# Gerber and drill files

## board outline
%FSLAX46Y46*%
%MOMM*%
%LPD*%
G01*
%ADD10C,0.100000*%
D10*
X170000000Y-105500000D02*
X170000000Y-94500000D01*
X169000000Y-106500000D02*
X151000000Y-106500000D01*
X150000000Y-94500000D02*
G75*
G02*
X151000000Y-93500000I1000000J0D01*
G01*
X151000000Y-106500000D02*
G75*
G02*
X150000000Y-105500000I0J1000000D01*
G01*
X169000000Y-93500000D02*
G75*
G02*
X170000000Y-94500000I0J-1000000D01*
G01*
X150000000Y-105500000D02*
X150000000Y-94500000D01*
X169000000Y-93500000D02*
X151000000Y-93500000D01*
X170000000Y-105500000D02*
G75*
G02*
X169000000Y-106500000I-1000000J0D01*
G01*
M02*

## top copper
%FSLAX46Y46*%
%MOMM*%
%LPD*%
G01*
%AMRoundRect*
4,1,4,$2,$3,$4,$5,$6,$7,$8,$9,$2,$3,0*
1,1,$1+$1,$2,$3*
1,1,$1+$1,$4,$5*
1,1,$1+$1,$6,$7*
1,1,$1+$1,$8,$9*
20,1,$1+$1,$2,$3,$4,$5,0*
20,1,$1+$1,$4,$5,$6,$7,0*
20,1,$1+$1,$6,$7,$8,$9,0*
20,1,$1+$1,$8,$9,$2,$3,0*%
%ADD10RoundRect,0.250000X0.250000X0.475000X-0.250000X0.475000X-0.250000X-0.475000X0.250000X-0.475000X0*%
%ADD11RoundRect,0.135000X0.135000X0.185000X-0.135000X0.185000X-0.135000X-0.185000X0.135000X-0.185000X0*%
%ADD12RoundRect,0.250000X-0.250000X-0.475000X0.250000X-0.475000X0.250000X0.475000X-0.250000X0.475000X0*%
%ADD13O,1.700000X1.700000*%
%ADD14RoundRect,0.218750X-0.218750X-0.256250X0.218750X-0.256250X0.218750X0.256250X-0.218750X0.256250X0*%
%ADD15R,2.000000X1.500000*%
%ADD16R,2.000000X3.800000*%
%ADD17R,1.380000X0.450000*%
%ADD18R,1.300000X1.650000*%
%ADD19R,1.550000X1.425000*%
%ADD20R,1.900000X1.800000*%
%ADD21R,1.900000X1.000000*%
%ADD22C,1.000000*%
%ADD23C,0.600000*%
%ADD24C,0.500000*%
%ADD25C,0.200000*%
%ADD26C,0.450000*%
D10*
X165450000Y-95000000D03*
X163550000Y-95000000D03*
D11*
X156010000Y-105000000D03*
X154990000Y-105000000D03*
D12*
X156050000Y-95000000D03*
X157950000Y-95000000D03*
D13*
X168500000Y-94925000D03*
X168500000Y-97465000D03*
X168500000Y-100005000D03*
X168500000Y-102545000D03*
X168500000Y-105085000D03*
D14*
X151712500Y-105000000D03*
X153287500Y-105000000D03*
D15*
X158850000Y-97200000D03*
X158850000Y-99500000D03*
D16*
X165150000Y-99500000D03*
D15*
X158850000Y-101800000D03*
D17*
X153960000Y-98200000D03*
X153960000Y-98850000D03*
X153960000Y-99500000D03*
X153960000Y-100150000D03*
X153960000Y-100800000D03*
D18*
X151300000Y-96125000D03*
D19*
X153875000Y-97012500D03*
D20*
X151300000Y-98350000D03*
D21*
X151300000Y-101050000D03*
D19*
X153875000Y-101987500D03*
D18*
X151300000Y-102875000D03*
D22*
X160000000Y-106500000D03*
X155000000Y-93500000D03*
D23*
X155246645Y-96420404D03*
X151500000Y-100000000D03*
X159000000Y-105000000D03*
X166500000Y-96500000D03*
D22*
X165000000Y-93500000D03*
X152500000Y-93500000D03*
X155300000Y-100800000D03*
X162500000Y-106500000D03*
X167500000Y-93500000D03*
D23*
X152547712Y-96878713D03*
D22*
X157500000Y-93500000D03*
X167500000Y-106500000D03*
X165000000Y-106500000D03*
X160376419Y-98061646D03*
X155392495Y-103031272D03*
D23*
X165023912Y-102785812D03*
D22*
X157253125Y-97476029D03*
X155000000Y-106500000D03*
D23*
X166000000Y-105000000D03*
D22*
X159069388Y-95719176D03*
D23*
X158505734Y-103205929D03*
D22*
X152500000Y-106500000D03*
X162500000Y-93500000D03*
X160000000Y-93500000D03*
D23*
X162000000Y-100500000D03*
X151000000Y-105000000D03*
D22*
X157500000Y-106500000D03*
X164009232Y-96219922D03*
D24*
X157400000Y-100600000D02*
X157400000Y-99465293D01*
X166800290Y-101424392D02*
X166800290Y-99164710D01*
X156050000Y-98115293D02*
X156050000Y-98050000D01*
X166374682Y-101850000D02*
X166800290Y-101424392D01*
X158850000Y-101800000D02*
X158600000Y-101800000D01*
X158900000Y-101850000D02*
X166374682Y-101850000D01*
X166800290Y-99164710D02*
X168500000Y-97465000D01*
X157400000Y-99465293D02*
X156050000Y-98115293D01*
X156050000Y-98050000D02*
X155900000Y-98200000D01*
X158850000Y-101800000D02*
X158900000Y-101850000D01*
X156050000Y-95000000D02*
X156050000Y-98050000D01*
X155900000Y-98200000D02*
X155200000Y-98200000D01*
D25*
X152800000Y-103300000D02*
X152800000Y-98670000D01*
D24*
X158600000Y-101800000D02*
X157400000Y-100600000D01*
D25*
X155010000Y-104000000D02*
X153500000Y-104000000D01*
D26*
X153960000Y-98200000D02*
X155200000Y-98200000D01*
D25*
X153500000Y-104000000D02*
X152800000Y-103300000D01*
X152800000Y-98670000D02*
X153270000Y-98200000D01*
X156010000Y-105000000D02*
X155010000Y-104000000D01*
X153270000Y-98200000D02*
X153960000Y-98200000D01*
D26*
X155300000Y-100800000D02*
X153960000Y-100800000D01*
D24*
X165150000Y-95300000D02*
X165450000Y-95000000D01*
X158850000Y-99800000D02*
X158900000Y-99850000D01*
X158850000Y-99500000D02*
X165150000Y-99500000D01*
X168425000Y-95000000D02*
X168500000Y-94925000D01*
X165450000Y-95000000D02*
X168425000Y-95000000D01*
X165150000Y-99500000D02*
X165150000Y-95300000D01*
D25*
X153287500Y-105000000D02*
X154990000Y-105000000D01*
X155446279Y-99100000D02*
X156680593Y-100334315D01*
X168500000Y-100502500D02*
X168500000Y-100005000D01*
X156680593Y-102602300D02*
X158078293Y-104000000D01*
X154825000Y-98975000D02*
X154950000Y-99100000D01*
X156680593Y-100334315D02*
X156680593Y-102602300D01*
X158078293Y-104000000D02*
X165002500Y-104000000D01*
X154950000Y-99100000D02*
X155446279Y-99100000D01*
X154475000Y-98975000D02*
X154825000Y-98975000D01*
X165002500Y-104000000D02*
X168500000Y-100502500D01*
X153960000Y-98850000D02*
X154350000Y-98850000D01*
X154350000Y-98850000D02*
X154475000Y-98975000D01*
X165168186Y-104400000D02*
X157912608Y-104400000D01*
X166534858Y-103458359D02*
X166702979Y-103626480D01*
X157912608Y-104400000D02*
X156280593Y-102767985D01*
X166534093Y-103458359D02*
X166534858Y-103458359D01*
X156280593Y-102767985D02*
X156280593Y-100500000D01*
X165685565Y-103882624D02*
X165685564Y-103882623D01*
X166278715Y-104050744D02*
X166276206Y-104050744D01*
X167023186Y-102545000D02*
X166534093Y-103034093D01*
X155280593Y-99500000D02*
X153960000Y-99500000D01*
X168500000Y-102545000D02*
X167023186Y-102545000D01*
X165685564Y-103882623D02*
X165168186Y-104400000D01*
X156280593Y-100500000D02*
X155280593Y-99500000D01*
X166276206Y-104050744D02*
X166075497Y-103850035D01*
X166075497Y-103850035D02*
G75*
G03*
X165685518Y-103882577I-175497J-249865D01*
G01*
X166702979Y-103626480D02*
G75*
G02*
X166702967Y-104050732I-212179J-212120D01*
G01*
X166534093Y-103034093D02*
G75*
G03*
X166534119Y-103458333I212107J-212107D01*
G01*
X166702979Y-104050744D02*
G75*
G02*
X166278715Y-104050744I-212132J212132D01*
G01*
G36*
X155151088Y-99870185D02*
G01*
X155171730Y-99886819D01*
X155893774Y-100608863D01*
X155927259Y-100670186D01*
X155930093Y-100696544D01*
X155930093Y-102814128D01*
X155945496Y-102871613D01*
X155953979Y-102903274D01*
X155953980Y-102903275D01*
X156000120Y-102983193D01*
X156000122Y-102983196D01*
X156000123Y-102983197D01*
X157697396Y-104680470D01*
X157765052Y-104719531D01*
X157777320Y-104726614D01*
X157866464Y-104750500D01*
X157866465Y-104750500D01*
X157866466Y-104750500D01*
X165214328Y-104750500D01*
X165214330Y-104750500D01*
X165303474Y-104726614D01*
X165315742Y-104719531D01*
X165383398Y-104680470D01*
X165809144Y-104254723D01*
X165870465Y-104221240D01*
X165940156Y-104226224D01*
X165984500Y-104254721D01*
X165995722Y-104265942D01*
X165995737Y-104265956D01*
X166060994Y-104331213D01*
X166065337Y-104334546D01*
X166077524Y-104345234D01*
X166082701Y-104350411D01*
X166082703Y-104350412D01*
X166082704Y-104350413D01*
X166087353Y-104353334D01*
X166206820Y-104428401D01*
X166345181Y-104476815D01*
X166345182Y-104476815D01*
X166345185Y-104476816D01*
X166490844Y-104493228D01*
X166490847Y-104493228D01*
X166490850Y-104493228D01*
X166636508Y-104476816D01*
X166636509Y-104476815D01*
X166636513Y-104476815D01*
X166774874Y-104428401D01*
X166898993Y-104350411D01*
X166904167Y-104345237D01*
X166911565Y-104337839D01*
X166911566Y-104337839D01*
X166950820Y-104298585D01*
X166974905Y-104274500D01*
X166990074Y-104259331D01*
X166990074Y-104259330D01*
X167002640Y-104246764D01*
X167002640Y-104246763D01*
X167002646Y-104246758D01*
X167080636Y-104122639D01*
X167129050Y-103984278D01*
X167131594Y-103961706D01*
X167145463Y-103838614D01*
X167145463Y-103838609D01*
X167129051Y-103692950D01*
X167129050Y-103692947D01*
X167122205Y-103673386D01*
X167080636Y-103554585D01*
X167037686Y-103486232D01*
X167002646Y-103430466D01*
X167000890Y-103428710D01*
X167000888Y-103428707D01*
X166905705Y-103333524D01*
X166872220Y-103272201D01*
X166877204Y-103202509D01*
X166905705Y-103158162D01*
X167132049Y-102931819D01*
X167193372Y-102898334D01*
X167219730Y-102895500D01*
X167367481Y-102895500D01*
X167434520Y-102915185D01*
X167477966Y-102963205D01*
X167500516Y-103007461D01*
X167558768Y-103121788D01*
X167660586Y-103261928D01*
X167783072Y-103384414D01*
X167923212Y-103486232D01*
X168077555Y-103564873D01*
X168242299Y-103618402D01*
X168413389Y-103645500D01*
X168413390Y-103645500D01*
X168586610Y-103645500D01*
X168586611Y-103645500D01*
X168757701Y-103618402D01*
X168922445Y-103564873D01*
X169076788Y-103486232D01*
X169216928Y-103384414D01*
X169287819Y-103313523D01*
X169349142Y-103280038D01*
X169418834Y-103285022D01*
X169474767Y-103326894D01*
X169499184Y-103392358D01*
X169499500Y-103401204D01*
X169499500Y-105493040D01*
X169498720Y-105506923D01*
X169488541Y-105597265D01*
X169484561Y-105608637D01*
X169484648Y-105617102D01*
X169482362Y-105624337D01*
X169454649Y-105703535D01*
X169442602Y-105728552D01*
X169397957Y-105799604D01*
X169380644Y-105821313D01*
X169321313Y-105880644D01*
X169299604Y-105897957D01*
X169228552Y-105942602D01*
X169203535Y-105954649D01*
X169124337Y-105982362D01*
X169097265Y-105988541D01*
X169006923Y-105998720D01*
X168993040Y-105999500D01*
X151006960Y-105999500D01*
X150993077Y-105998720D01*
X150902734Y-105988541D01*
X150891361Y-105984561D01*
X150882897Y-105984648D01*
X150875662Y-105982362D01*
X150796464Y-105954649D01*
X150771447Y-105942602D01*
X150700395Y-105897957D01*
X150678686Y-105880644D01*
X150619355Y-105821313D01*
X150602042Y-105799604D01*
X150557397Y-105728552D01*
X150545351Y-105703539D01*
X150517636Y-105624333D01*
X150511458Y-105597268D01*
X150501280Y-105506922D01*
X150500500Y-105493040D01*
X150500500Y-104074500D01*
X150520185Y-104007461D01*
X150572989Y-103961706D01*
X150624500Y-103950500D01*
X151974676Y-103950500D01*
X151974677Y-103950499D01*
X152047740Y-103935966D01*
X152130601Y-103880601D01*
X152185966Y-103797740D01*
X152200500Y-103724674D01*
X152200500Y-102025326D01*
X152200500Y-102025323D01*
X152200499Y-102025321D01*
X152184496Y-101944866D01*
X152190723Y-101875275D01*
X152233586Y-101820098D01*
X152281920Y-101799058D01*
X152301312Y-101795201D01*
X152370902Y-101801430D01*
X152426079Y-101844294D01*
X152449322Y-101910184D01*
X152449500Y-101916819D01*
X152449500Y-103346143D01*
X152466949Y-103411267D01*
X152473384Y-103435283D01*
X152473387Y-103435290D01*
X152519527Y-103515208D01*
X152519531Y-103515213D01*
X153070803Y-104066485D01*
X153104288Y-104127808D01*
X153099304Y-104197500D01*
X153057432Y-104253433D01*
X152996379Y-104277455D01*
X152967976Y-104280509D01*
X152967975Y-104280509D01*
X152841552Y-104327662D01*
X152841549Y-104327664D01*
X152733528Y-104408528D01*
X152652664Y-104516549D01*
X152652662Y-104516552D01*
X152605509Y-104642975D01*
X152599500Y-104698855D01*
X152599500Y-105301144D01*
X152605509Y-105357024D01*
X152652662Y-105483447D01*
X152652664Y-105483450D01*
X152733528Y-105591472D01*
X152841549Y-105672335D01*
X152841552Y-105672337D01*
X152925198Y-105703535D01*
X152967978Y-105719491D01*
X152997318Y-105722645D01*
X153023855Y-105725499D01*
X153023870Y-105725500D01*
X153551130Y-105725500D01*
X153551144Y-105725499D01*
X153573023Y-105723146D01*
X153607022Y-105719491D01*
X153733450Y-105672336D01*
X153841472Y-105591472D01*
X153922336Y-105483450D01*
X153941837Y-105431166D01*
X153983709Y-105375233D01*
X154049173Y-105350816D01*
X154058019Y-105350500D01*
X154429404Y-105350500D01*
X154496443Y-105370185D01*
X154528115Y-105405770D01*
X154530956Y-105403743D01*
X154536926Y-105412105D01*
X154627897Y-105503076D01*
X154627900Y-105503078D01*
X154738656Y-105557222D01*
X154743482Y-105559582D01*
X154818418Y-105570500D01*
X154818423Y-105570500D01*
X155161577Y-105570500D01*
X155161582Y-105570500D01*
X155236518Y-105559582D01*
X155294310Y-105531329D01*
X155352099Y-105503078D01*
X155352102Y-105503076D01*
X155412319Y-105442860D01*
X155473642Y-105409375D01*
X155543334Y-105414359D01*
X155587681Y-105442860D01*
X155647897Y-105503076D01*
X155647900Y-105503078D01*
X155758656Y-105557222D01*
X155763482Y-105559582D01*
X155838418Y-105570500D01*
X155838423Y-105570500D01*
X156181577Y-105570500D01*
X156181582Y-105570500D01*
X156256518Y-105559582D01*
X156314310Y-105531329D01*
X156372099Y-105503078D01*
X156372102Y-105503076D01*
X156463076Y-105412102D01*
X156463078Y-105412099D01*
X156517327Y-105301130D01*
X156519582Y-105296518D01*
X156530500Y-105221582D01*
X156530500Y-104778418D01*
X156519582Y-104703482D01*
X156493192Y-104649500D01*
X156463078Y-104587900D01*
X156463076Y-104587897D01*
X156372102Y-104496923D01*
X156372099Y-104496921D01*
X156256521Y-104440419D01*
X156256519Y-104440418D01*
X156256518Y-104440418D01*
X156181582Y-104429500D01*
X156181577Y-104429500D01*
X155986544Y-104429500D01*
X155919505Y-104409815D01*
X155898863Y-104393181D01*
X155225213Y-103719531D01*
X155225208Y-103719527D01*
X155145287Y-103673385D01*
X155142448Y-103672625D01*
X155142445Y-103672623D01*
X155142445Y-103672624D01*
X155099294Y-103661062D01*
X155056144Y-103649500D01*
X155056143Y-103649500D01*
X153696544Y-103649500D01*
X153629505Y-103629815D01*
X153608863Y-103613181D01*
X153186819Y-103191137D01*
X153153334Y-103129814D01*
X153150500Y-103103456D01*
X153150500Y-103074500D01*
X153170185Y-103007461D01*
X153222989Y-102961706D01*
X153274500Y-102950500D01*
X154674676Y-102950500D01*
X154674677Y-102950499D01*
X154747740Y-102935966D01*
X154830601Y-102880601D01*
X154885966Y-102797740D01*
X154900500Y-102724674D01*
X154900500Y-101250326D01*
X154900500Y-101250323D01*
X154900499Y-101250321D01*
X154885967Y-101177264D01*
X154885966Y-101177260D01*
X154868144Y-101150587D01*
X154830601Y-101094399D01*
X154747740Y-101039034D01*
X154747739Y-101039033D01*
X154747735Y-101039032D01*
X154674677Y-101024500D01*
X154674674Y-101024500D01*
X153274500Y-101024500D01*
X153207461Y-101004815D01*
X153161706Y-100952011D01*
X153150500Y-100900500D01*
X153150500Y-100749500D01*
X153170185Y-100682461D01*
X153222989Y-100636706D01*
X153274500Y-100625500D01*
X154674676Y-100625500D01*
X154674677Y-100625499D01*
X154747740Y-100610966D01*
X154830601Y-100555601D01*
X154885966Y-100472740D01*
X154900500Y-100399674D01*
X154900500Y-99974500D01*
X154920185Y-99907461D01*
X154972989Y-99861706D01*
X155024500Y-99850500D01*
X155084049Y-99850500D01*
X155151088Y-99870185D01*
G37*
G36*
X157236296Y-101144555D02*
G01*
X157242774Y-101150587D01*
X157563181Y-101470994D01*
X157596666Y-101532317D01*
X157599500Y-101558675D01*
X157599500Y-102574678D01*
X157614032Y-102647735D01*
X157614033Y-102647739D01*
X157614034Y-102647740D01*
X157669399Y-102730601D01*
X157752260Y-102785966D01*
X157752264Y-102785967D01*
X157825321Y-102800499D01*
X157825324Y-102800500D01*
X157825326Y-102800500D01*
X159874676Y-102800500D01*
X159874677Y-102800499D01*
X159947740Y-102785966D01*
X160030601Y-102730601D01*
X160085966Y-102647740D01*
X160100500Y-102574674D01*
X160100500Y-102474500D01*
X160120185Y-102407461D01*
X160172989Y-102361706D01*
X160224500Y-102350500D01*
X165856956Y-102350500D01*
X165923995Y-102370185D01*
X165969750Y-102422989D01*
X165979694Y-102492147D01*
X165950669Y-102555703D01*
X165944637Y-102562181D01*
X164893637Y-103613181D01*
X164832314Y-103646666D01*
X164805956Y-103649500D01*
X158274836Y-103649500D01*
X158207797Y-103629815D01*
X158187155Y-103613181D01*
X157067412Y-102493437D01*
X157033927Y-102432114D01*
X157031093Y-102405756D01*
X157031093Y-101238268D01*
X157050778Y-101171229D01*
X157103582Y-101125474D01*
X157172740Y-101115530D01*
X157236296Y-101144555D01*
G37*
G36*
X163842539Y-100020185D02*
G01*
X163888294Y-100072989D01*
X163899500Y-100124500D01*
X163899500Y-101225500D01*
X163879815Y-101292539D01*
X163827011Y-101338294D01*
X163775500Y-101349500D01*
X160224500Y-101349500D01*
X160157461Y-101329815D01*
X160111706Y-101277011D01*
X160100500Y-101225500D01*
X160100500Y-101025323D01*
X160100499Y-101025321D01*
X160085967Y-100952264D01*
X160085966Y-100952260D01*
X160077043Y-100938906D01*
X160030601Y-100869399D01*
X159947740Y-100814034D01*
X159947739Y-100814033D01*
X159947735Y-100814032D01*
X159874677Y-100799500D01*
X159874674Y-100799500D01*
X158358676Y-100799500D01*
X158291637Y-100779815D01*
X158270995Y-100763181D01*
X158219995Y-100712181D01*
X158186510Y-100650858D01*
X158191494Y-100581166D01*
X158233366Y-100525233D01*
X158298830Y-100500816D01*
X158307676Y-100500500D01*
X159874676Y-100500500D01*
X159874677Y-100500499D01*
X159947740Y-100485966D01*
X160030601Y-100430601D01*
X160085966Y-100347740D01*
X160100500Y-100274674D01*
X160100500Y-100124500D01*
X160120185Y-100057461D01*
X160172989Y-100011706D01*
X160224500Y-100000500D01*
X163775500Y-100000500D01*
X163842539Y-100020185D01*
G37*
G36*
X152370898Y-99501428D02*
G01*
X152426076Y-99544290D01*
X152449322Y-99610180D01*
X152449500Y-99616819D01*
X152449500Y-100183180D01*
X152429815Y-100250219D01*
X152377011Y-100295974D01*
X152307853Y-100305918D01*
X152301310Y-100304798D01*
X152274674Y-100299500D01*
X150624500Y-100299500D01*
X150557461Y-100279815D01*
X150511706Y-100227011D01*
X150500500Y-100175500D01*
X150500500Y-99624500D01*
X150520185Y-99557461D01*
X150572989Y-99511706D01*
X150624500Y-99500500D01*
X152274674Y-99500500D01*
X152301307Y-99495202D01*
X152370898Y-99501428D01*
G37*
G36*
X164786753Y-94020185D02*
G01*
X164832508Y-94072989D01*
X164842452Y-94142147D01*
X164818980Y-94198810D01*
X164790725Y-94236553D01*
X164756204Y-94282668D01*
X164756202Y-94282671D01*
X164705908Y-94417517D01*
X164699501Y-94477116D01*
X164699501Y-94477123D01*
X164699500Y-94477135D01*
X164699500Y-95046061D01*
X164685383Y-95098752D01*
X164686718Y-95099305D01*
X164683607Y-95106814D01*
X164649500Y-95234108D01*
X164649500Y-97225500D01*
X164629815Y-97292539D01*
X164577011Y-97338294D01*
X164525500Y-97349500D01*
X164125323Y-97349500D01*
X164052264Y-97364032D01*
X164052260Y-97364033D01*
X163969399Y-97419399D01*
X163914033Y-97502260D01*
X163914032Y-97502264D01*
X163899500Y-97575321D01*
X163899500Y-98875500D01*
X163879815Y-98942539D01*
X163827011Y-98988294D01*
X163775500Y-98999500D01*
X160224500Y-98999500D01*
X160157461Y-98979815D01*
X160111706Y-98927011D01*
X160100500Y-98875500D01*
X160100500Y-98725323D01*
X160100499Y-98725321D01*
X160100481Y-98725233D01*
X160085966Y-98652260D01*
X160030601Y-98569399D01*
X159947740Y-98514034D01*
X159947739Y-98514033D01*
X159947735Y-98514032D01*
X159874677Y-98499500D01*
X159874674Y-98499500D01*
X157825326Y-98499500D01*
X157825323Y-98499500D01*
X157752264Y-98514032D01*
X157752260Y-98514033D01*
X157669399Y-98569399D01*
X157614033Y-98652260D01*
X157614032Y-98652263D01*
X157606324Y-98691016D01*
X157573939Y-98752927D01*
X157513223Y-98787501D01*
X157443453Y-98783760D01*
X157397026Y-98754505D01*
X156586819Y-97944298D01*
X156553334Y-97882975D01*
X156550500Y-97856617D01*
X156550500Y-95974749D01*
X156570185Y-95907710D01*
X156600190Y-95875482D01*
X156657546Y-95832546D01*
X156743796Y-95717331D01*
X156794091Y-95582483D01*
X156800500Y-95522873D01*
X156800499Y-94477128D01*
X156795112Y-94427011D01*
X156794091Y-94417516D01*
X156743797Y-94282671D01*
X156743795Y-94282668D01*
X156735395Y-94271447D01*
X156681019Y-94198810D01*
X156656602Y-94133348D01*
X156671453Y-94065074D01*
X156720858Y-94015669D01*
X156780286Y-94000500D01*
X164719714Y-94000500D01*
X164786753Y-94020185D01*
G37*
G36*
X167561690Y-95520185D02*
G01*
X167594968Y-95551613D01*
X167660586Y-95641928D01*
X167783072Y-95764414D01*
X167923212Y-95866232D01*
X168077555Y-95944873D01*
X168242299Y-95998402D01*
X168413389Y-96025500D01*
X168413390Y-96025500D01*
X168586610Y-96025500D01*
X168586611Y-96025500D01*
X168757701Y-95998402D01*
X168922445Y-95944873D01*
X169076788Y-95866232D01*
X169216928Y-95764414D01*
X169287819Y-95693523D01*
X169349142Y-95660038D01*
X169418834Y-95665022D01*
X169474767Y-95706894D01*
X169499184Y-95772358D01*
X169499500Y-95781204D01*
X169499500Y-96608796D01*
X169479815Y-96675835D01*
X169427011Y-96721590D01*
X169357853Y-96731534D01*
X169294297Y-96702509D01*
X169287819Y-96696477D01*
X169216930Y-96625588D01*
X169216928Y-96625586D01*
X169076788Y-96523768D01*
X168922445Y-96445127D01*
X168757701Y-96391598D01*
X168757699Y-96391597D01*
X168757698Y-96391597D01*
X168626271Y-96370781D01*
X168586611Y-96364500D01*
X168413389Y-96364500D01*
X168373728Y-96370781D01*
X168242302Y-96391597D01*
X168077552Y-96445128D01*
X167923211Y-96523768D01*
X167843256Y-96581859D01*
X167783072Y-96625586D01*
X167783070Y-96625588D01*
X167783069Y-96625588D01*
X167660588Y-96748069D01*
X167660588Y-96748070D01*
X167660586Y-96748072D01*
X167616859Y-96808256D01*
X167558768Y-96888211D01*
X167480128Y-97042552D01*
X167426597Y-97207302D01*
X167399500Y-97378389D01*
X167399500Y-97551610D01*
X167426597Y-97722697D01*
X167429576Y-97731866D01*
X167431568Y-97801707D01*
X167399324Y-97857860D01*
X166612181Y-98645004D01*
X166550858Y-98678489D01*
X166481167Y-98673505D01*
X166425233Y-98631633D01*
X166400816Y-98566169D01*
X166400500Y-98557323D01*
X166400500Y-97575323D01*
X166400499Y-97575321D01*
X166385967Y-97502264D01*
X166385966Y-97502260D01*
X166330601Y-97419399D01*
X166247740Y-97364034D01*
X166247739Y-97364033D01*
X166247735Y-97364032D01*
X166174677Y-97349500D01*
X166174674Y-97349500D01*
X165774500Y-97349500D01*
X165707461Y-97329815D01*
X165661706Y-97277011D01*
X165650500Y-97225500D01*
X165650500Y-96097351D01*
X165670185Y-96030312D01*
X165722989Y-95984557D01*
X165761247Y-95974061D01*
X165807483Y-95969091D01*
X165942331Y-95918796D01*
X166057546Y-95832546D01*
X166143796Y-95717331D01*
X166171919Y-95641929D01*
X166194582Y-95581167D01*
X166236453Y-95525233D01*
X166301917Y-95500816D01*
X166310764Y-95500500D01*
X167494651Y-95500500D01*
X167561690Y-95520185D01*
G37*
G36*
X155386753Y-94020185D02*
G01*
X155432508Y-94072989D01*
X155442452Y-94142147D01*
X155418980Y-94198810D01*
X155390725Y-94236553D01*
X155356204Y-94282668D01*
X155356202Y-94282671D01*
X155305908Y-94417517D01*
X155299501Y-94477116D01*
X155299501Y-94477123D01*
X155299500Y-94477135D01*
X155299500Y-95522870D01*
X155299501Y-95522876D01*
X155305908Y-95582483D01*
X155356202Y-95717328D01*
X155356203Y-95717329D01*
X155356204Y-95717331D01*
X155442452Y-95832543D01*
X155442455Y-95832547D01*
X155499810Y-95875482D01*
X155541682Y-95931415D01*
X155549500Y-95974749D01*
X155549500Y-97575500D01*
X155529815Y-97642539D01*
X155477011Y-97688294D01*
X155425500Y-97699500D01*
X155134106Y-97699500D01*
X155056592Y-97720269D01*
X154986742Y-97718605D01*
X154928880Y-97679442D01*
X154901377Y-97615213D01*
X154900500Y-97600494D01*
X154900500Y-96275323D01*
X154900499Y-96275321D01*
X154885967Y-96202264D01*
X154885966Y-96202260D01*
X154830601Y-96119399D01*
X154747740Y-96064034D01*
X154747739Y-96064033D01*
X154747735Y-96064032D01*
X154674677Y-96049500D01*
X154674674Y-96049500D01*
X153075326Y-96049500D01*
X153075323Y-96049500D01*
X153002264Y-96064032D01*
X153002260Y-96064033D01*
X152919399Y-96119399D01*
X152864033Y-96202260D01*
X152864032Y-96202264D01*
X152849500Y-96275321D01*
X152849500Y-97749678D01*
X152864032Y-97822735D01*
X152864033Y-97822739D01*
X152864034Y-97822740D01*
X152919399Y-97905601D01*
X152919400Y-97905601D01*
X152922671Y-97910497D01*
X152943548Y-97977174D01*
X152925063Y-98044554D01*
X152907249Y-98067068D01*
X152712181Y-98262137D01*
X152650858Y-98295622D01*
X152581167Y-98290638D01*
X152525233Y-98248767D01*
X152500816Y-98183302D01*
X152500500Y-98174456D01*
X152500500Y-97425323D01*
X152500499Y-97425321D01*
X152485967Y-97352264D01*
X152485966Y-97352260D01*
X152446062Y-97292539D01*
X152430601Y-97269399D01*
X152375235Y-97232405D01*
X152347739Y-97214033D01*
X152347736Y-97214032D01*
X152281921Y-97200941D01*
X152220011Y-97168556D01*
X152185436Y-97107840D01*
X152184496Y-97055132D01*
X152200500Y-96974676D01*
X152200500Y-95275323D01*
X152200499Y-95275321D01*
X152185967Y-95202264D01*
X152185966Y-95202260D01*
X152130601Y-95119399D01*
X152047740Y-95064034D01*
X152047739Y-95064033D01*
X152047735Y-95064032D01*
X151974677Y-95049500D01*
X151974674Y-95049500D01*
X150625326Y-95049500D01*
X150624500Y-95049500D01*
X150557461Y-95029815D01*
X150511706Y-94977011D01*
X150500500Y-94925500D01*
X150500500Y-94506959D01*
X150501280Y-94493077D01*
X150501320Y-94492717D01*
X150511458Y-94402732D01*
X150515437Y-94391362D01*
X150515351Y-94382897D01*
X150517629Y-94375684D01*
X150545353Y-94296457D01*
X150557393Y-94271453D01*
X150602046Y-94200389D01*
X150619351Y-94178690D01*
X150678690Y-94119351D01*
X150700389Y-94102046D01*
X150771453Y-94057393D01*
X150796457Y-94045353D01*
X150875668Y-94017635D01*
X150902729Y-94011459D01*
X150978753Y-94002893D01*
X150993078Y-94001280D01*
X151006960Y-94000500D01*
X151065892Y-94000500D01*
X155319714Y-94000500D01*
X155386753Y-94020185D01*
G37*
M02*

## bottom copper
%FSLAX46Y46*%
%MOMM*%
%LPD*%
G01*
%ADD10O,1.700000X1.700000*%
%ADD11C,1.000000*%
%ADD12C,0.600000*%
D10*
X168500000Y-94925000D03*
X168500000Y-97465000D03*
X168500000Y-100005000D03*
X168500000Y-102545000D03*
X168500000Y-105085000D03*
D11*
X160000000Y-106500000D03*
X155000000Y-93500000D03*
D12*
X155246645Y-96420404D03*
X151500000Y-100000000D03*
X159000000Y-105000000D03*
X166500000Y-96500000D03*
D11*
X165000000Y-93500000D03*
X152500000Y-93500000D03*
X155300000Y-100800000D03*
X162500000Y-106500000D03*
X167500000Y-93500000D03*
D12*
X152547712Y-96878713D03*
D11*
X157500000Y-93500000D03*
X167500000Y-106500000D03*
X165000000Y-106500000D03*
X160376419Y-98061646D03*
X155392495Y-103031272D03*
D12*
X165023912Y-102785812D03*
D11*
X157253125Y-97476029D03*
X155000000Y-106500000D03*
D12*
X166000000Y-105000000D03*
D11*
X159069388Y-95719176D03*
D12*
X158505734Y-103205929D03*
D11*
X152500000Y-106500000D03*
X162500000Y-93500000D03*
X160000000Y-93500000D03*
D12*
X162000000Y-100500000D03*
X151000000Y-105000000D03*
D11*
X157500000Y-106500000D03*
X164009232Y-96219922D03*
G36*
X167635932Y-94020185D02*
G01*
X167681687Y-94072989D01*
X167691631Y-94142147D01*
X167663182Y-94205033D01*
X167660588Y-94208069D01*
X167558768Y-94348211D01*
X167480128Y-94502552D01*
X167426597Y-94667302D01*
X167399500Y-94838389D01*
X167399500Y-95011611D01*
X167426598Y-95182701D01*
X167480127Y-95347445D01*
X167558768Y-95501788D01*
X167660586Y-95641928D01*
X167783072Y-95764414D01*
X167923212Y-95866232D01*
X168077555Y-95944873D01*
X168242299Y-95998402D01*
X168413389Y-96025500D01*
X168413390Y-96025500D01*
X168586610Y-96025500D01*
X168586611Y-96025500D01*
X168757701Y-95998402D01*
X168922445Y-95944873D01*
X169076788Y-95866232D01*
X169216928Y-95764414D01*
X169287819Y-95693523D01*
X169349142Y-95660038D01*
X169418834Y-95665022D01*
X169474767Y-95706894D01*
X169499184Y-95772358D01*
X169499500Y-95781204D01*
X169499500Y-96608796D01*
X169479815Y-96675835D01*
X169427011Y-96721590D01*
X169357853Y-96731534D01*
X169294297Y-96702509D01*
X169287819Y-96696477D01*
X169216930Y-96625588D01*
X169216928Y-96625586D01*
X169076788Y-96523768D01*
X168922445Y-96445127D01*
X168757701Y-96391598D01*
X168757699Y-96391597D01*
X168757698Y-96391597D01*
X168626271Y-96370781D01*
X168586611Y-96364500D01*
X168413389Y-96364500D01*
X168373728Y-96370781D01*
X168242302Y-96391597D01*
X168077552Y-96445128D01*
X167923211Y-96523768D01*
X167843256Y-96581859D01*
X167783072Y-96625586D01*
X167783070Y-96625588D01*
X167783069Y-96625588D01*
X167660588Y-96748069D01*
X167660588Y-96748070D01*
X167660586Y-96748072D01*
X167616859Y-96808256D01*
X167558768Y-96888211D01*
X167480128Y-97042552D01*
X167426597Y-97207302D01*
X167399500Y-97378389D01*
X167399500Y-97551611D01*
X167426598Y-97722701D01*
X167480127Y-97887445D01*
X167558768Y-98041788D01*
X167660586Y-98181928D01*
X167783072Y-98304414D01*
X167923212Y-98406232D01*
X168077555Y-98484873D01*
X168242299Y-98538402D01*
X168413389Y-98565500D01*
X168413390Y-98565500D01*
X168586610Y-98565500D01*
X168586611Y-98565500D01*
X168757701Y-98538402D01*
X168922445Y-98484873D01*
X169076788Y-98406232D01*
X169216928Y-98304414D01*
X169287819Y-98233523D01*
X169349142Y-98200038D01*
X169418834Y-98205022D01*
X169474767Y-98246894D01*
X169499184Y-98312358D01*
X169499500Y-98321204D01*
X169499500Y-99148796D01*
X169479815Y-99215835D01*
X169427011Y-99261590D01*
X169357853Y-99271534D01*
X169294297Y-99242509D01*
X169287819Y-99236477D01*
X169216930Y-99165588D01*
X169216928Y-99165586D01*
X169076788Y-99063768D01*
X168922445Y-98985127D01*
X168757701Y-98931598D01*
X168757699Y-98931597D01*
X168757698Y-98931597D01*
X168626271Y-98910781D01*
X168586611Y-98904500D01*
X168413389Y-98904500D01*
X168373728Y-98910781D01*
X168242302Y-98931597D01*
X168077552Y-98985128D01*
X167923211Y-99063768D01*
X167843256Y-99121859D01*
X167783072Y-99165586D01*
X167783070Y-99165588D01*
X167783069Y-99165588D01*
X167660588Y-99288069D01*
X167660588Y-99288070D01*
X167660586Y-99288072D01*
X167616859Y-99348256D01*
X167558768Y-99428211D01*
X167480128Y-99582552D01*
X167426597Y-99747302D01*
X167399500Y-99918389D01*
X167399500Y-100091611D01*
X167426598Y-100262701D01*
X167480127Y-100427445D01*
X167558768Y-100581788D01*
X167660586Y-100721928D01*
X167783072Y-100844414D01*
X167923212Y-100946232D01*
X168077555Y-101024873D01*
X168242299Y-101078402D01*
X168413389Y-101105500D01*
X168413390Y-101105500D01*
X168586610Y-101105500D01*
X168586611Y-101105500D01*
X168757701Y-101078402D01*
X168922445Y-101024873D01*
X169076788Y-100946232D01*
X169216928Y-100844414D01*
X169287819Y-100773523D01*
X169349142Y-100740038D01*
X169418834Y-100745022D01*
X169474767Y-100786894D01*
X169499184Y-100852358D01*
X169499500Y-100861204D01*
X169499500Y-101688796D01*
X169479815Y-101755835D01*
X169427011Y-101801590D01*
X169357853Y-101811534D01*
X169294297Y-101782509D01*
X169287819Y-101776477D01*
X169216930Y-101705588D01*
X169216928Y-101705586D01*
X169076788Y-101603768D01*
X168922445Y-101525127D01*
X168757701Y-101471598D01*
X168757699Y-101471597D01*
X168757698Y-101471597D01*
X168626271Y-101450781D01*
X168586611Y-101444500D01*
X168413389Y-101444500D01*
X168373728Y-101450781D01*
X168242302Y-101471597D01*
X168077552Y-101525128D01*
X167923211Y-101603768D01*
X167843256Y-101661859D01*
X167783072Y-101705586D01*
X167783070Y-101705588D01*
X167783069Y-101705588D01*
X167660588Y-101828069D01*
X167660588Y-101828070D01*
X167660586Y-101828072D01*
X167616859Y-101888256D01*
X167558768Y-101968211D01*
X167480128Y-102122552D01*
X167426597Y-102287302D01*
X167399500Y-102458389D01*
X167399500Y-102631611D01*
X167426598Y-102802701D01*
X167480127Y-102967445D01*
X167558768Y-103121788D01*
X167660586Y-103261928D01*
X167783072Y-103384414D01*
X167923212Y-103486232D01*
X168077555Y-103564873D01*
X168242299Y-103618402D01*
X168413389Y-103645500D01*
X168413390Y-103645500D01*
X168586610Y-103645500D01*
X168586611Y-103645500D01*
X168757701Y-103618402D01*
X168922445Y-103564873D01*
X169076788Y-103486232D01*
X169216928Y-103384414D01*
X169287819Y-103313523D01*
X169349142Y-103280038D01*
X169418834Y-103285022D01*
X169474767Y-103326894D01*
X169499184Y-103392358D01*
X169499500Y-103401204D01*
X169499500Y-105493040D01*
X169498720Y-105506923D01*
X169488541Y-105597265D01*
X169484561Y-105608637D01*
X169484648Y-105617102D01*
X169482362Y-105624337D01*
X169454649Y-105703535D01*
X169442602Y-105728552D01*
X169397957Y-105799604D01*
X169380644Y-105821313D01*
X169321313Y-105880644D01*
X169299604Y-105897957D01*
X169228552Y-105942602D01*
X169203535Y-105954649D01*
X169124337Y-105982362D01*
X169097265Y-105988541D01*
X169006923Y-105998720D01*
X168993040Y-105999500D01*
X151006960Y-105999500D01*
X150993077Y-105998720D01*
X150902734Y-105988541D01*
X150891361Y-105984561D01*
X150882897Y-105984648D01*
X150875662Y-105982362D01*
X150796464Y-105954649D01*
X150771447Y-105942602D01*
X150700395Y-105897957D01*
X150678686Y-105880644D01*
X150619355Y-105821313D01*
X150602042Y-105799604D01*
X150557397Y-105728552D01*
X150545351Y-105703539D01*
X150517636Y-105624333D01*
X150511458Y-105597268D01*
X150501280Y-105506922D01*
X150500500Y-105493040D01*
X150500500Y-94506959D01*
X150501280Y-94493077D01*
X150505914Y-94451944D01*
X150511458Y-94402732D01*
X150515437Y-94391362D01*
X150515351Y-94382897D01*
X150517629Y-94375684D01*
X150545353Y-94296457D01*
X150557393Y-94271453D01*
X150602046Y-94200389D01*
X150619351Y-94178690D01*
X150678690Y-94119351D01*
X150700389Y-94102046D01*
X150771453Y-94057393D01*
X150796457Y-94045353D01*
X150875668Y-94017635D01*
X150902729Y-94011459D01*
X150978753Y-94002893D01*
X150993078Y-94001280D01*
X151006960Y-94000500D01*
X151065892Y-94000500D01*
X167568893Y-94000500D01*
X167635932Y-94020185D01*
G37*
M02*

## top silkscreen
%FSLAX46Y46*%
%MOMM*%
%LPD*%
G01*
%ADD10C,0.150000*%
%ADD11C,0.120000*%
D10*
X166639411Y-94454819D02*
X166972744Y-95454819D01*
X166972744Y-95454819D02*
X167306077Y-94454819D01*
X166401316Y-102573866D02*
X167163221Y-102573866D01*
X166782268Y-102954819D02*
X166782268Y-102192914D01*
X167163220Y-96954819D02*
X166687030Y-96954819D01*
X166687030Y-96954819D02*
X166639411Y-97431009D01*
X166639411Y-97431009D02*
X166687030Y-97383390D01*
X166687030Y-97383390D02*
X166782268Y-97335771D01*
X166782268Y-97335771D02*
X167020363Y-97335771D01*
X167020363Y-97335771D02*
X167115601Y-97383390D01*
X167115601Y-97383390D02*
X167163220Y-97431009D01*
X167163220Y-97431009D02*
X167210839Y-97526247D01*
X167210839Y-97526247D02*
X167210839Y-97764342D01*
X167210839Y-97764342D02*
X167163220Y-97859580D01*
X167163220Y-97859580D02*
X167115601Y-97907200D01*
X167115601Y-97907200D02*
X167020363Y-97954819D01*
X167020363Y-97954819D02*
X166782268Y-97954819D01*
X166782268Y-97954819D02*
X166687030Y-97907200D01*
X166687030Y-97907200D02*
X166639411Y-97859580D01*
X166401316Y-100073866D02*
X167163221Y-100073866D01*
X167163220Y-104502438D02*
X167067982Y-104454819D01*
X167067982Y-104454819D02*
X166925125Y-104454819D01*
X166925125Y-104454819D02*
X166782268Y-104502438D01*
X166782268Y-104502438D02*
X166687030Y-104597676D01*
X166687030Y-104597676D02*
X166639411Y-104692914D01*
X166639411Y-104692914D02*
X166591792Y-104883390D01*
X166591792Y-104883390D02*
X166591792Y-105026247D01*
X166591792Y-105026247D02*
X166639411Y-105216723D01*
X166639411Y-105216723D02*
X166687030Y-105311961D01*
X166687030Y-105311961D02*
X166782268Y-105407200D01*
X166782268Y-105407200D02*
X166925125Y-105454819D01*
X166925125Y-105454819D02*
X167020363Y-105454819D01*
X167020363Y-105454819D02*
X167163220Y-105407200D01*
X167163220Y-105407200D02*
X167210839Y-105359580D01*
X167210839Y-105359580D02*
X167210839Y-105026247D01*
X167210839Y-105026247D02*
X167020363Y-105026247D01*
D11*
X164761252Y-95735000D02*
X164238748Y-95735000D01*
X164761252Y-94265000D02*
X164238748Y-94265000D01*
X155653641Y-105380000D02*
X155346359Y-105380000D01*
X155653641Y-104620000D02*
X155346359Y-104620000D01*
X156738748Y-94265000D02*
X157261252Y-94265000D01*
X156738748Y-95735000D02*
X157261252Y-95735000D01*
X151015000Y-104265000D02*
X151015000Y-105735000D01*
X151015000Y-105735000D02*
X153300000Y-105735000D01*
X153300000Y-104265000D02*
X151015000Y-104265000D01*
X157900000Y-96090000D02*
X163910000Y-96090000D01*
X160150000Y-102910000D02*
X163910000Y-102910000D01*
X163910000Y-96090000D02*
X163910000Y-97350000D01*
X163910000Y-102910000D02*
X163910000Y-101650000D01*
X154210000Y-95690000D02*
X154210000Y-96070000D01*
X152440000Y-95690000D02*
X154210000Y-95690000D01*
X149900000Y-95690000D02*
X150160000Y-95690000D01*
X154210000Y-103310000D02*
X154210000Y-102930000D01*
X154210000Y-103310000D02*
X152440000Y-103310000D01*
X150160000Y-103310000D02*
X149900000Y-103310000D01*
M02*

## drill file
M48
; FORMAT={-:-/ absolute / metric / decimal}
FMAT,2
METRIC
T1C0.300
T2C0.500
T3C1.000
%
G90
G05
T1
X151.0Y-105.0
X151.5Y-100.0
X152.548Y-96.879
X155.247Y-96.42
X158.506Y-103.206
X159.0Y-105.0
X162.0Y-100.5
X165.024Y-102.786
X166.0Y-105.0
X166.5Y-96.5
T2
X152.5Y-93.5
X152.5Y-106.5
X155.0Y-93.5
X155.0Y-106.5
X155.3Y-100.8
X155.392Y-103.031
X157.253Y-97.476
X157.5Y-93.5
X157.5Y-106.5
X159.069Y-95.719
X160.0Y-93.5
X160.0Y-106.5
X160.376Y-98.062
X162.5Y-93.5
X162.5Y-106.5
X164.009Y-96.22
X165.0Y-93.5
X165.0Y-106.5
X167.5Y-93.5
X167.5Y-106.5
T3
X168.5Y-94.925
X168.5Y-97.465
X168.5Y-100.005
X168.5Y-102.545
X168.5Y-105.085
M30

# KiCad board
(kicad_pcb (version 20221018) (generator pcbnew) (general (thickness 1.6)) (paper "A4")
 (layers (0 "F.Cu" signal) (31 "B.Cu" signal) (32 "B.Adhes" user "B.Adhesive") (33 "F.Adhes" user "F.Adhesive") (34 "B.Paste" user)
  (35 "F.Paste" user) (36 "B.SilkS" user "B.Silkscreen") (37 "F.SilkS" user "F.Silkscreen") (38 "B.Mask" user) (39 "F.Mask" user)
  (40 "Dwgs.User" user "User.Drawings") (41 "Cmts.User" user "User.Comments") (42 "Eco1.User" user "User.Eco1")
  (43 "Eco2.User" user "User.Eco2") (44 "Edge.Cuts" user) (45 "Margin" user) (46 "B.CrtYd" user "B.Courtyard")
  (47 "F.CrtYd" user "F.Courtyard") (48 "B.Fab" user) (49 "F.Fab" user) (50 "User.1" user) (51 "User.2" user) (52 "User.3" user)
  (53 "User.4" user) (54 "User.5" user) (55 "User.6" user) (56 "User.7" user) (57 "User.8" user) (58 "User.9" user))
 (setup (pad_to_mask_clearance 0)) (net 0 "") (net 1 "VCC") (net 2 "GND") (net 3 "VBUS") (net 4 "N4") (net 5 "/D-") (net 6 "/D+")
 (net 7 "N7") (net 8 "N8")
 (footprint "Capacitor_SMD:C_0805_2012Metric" (layer "F.Cu") (at 164.5 95 180)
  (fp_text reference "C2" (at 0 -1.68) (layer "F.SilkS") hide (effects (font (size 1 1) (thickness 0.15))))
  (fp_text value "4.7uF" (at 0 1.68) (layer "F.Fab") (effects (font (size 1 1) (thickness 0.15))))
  (fp_line (start -0.261252 -0.735) (end 0.261252 -0.735) (stroke (width 0.12) (type solid)) (layer "F.SilkS"))
  (fp_line (start -0.261252 0.735) (end 0.261252 0.735) (stroke (width 0.12) (type solid)) (layer "F.SilkS"))
  (pad "1" smd roundrect (at -0.95 0 180) (size 1 1.45) (layers "F.Cu" "F.Paste" "F.Mask") (roundrect_rratio 0.25) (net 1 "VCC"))
  (pad "2" smd roundrect (at 0.95 0 180) (size 1 1.45) (layers "F.Cu" "F.Paste" "F.Mask") (roundrect_rratio 0.25) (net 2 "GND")))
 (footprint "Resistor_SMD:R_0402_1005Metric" (layer "F.Cu") (at 155.5 105 180)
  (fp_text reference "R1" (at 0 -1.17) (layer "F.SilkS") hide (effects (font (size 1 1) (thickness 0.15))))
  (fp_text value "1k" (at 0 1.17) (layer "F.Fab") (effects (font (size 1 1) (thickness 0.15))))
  (fp_line (start -0.153641 -0.38) (end 0.153641 -0.38) (stroke (width 0.12) (type solid)) (layer "F.SilkS"))
  (fp_line (start -0.153641 0.38) (end 0.153641 0.38) (stroke (width 0.12) (type solid)) (layer "F.SilkS"))
  (pad "1" smd roundrect (at -0.51 0 180) (size 0.54 0.64) (layers "F.Cu" "F.Paste" "F.Mask") (roundrect_rratio 0.25) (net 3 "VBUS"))
  (pad "2" smd roundrect (at 0.51 0 180) (size 0.54 0.64) (layers "F.Cu" "F.Paste" "F.Mask") (roundrect_rratio 0.25) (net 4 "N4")))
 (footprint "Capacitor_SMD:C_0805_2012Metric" (layer "F.Cu") (at 157 95)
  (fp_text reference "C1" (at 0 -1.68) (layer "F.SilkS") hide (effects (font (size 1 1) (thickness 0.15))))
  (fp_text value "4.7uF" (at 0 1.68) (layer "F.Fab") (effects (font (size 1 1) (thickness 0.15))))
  (fp_line (start -0.261252 -0.735) (end 0.261252 -0.735) (stroke (width 0.12) (type solid)) (layer "F.SilkS"))
  (fp_line (start -0.261252 0.735) (end 0.261252 0.735) (stroke (width 0.12) (type solid)) (layer "F.SilkS"))
  (pad "1" smd roundrect (at -0.95 0) (size 1 1.45) (layers "F.Cu" "F.Paste" "F.Mask") (roundrect_rratio 0.25) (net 3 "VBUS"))
  (pad "2" smd roundrect (at 0.95 0) (size 1 1.45) (layers "F.Cu" "F.Paste" "F.Mask") (roundrect_rratio 0.25) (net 2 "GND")))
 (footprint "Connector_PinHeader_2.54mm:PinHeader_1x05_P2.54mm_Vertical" (layer "F.Cu") (at 168.5 94.925)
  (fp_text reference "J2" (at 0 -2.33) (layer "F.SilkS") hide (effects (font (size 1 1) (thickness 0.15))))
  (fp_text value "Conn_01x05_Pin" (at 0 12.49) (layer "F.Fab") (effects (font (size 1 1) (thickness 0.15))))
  (pad "1" thru_hole oval (at 0 0) (size 1.7 1.7) (drill 1) (layers "*.Cu" "*.Mask") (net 1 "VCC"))
  (pad "2" thru_hole oval (at 0 2.54) (size 1.7 1.7) (drill 1) (layers "*.Cu" "*.Mask") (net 3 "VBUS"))
  (pad "3" thru_hole oval (at 0 5.08) (size 1.7 1.7) (drill 1) (layers "*.Cu" "*.Mask") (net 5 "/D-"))
  (pad "4" thru_hole oval (at 0 7.62) (size 1.7 1.7) (drill 1) (layers "*.Cu" "*.Mask") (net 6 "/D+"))
  (pad "5" thru_hole oval (at 0 10.16) (size 1.7 1.7) (drill 1) (layers "*.Cu" "*.Mask") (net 2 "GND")))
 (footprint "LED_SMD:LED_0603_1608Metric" (layer "F.Cu") (at 152.5 105)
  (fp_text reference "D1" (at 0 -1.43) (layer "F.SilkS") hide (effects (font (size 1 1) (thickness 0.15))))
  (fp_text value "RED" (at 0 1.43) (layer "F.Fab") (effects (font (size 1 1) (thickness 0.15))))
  (fp_line (start -1.485 -0.735) (end -1.485 0.735) (stroke (width 0.12) (type solid)) (layer "F.SilkS"))
  (fp_line (start -1.485 0.735) (end 0.8 0.735) (stroke (width 0.12) (type solid)) (layer "F.SilkS"))
  (fp_line (start 0.8 -0.735) (end -1.485 -0.735) (stroke (width 0.12) (type solid)) (layer "F.SilkS"))
  (pad "1" smd roundrect (at -0.7875 0) (size 0.875 0.95) (layers "F.Cu" "F.Paste" "F.Mask") (roundrect_rratio 0.25) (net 2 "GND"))
  (pad "2" smd roundrect (at 0.7875 0) (size 0.875 0.95) (layers "F.Cu" "F.Paste" "F.Mask") (roundrect_rratio 0.25) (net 4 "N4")))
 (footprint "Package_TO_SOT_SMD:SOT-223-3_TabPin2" (layer "F.Cu") (at 162 99.5)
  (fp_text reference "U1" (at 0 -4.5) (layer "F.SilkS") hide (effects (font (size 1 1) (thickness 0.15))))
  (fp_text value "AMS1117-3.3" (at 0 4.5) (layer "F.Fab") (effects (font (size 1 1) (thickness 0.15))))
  (fp_line (start -4.1 -3.41) (end 1.91 -3.41) (stroke (width 0.12) (type solid)) (layer "F.SilkS"))
  (fp_line (start -1.85 3.41) (end 1.91 3.41) (stroke (width 0.12) (type solid)) (layer "F.SilkS"))
  (fp_line (start 1.91 -3.41) (end 1.91 -2.15) (stroke (width 0.12) (type solid)) (layer "F.SilkS"))
  (fp_line (start 1.91 3.41) (end 1.91 2.15) (stroke (width 0.12) (type solid)) (layer "F.SilkS"))
  (pad "1" smd rect (at -3.15 -2.3) (size 2 1.5) (layers "F.Cu" "F.Paste" "F.Mask") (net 2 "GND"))
  (pad "2" smd rect (at -3.15 0) (size 2 1.5) (layers "F.Cu" "F.Paste" "F.Mask") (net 1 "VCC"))
  (pad "2" smd rect (at 3.15 0) (size 2 3.8) (layers "F.Cu" "F.Paste" "F.Mask") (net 1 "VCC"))
  (pad "3" smd rect (at -3.15 2.3) (size 2 1.5) (layers "F.Cu" "F.Paste" "F.Mask") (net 3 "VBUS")))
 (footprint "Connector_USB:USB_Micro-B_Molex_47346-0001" (layer "F.Cu") (at 152.5 99.5 -90)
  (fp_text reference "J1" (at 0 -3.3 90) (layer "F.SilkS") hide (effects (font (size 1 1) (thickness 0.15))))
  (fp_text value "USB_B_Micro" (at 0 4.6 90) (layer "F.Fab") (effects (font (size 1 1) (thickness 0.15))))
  (fp_line (start -3.81 -1.71) (end -3.43 -1.71) (stroke (width 0.12) (type solid)) (layer "F.SilkS"))
  (fp_line (start -3.81 0.06) (end -3.81 -1.71) (stroke (width 0.12) (type solid)) (layer "F.SilkS"))
  (fp_line (start -3.81 2.6) (end -3.81 2.34) (stroke (width 0.12) (type solid)) (layer "F.SilkS"))
  (fp_line (start 3.81 -1.71) (end 3.43 -1.71) (stroke (width 0.12) (type solid)) (layer "F.SilkS"))
  (fp_line (start 3.81 -1.71) (end 3.81 0.06) (stroke (width 0.12) (type solid)) (layer "F.SilkS"))
  (fp_line (start 3.81 2.34) (end 3.81 2.6) (stroke (width 0.12) (type solid)) (layer "F.SilkS"))
  (pad "1" smd rect (at -1.3 -1.46 270) (size 0.45 1.38) (layers "F.Cu" "F.Paste" "F.Mask") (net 3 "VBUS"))
  (pad "2" smd rect (at -0.65 -1.46 270) (size 0.45 1.38) (layers "F.Cu" "F.Paste" "F.Mask") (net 5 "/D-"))
  (pad "3" smd rect (at 0 -1.46 270) (size 0.45 1.38) (layers "F.Cu" "F.Paste" "F.Mask") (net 6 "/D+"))
  (pad "4" smd rect (at 0.65 -1.46 270) (size 0.45 1.38) (layers "F.Cu" "F.Paste" "F.Mask") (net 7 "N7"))
  (pad "5" smd rect (at 1.3 -1.46 270) (size 0.45 1.38) (layers "F.Cu" "F.Paste" "F.Mask") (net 2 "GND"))
  (pad "6" smd rect (at -3.375 1.2 270) (size 1.65 1.3) (layers "F.Cu" "F.Paste" "F.Mask") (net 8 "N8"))
  (pad "6" smd rect (at -2.4875 -1.375 270) (size 1.425 1.55) (layers "F.Cu" "F.Paste" "F.Mask") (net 8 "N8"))
  (pad "6" smd rect (at -1.15 1.2 270) (size 1.8 1.9) (layers "F.Cu" "F.Paste" "F.Mask") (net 8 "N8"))
  (pad "6" smd rect (at 1.55 1.2 270) (size 1 1.9) (layers "F.Cu" "F.Paste" "F.Mask") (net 8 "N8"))
  (pad "6" smd rect (at 2.4875 -1.375 270) (size 1.425 1.55) (layers "F.Cu" "F.Paste" "F.Mask") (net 8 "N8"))
  (pad "6" smd rect (at 3.375 1.2 270) (size 1.65 1.3) (layers "F.Cu" "F.Paste" "F.Mask") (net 8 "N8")))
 (gr_line (start 170 105.5) (end 170 94.5) (stroke (width 0.1) (type default)) (layer "Edge.Cuts"))
 (gr_line (start 169 106.5) (end 151 106.5) (stroke (width 0.1) (type default)) (layer "Edge.Cuts"))
 (gr_arc (start 150 94.5) (mid 150.292893 93.792893) (end 151 93.5) (stroke (width 0.1) (type default)) (layer "Edge.Cuts"))
 (gr_arc (start 151 106.5) (mid 150.292893 106.207107) (end 150 105.5) (stroke (width 0.1) (type default)) (layer "Edge.Cuts"))
 (gr_arc (start 169 93.5) (mid 169.707107 93.792893) (end 170 94.5) (stroke (width 0.1) (type default)) (layer "Edge.Cuts"))
 (gr_line (start 150 105.5) (end 150 94.5) (stroke (width 0.1) (type default)) (layer "Edge.Cuts"))
 (gr_line (start 169 93.5) (end 151 93.5) (stroke (width 0.1) (type default)) (layer "Edge.Cuts"))
 (gr_arc (start 170 105.5) (mid 169.707107 106.207107) (end 169 106.5) (stroke (width 0.1) (type default)) (layer "Edge.Cuts"))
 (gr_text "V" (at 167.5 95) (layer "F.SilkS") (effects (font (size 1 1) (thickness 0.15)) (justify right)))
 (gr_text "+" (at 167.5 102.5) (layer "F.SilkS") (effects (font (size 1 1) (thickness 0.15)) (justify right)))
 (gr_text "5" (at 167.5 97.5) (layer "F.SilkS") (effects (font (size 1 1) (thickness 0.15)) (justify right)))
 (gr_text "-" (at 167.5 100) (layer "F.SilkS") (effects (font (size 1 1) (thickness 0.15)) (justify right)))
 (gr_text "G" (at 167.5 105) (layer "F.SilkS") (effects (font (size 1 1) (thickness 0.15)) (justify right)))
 (segment (start 157.4 100.6) (end 157.4 99.465293) (width 0.5) (layer "F.Cu") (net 3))
 (segment (start 166.80029 101.424392) (end 166.80029 99.16471) (width 0.5) (layer "F.Cu") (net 3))
 (segment (start 156.05 98.115293) (end 156.05 98.05) (width 0.5) (layer "F.Cu") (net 3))
 (segment (start 166.374682 101.85) (end 166.80029 101.424392) (width 0.5) (layer "F.Cu") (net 3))
 (segment (start 158.85 101.8) (end 158.6 101.8) (width 0.5) (layer "F.Cu") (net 3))
 (segment (start 158.9 101.85) (end 166.374682 101.85) (width 0.5) (layer "F.Cu") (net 3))
 (segment (start 166.80029 99.16471) (end 168.5 97.465) (width 0.5) (layer "F.Cu") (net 3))
 (segment (start 157.4 99.465293) (end 156.05 98.115293) (width 0.5) (layer "F.Cu") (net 3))
 (segment (start 156.05 98.05) (end 155.9 98.2) (width 0.5) (layer "F.Cu") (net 3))
 (segment (start 158.85 101.8) (end 158.9 101.85) (width 0.5) (layer "F.Cu") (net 3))
 (segment (start 156.05 95) (end 156.05 98.05) (width 0.5) (layer "F.Cu") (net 3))
 (segment (start 155.9 98.2) (end 155.2 98.2) (width 0.5) (layer "F.Cu") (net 3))
 (segment (start 152.8 103.3) (end 152.8 98.67) (width 0.2) (layer "F.Cu") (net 3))
 (segment (start 158.6 101.8) (end 157.4 100.6) (width 0.5) (layer "F.Cu") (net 3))
 (segment (start 155.01 104) (end 153.5 104) (width 0.2) (layer "F.Cu") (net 3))
 (segment (start 153.96 98.2) (end 155.2 98.2) (width 0.45) (layer "F.Cu") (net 3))
 (segment (start 153.5 104) (end 152.8 103.3) (width 0.2) (layer "F.Cu") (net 3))
 (segment (start 152.8 98.67) (end 153.27 98.2) (width 0.2) (layer "F.Cu") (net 3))
 (segment (start 156.01 105) (end 155.01 104) (width 0.2) (layer "F.Cu") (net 3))
 (segment (start 153.27 98.2) (end 153.96 98.2) (width 0.2) (layer "F.Cu") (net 3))
 (segment (start 155.3 100.8) (end 153.96 100.8) (width 0.45) (layer "F.Cu") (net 2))
 (via (at 160 106.5) (size 1) (drill 0.5) (layers "F.Cu" "B.Cu") (free) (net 2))
 (via (at 155 93.5) (size 1) (drill 0.5) (layers "F.Cu" "B.Cu") (free) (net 2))
 (via (at 155.246645 96.420404) (size 0.6) (drill 0.3) (layers "F.Cu" "B.Cu") (free) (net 2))
 (via (at 151.5 100) (size 0.6) (drill 0.3) (layers "F.Cu" "B.Cu") (free) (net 2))
 (via (at 159 105) (size 0.6) (drill 0.3) (layers "F.Cu" "B.Cu") (free) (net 2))
 (via (at 166.5 96.5) (size 0.6) (drill 0.3) (layers "F.Cu" "B.Cu") (free) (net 2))
 (via (at 165 93.5) (size 1) (drill 0.5) (layers "F.Cu" "B.Cu") (free) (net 2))
 (via (at 152.5 93.5) (size 1) (drill 0.5) (layers "F.Cu" "B.Cu") (free) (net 2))
 (via (at 155.3 100.8) (size 1) (drill 0.5) (layers "F.Cu" "B.Cu") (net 2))
 (via (at 162.5 106.5) (size 1) (drill 0.5) (layers "F.Cu" "B.Cu") (free) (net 2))
 (via (at 167.5 93.5) (size 1) (drill 0.5) (layers "F.Cu" "B.Cu") (free) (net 2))
 (via (at 152.547712 96.878713) (size 0.6) (drill 0.3) (layers "F.Cu" "B.Cu") (free) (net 2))
 (via (at 157.5 93.5) (size 1) (drill 0.5) (layers "F.Cu" "B.Cu") (free) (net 2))
 (via (at 167.5 106.5) (size 1) (drill 0.5) (layers "F.Cu" "B.Cu") (free) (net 2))
 (via (at 165 106.5) (size 1) (drill 0.5) (layers "F.Cu" "B.Cu") (free) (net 2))
 (via (at 160.376419 98.061646) (size 1) (drill 0.5) (layers "F.Cu" "B.Cu") (free) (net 2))
 (via (at 155.392495 103.031272) (size 1) (drill 0.5) (layers "F.Cu" "B.Cu") (free) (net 2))
 (via (at 165.023912 102.785812) (size 0.6) (drill 0.3) (layers "F.Cu" "B.Cu") (free) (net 2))
 (via (at 157.253125 97.476029) (size 1) (drill 0.5) (layers "F.Cu" "B.Cu") (free) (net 2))
 (via (at 155 106.5) (size 1) (drill 0.5) (layers "F.Cu" "B.Cu") (free) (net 2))
 (via (at 166 105) (size 0.6) (drill 0.3) (layers "F.Cu" "B.Cu") (free) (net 2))
 (via (at 159.069388 95.719176) (size 1) (drill 0.5) (layers "F.Cu" "B.Cu") (free) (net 2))
 (via (at 158.505734 103.205929) (size 0.6) (drill 0.3) (layers "F.Cu" "B.Cu") (free) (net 2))
 (via (at 152.5 106.5) (size 1) (drill 0.5) (layers "F.Cu" "B.Cu") (free) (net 2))
 (via (at 162.5 93.5) (size 1) (drill 0.5) (layers "F.Cu" "B.Cu") (free) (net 2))
 (via (at 160 93.5) (size 1) (drill 0.5) (layers "F.Cu" "B.Cu") (free) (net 2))
 (via (at 162 100.5) (size 0.6) (drill 0.3) (layers "F.Cu" "B.Cu") (free) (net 2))
 (via (at 151 105) (size 0.6) (drill 0.3) (layers "F.Cu" "B.Cu") (free) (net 2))
 (via (at 157.5 106.5) (size 1) (drill 0.5) (layers "F.Cu" "B.Cu") (free) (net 2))
 (via (at 164.009232 96.219922) (size 1) (drill 0.5) (layers "F.Cu" "B.Cu") (free) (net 2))
 (segment (start 165.15 95.3) (end 165.45 95) (width 0.5) (layer "F.Cu") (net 1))
 (segment (start 158.85 99.8) (end 158.9 99.85) (width 0.5) (layer "F.Cu") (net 1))
 (segment (start 158.85 99.5) (end 165.15 99.5) (width 0.5) (layer "F.Cu") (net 1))
 (segment (start 168.425 95) (end 168.5 94.925) (width 0.5) (layer "F.Cu") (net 1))
 (segment (start 165.45 95) (end 168.425 95) (width 0.5) (layer "F.Cu") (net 1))
 (segment (start 165.15 99.5) (end 165.15 95.3) (width 0.5) (layer "F.Cu") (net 1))
 (segment (start 153.2875 105) (end 154.99 105) (width 0.2) (layer "F.Cu") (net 4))
 (segment (start 155.446279 99.1) (end 156.680593 100.334315) (width 0.2) (layer "F.Cu") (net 5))
 (segment (start 168.5 100.5025) (end 168.5 100.005) (width 0.2) (layer "F.Cu") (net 5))
 (segment (start 156.680593 102.6023) (end 158.078293 104) (width 0.2) (layer "F.Cu") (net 5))
 (segment (start 154.825 98.975) (end 154.95 99.1) (width 0.2) (layer "F.Cu") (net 5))
 (segment (start 156.680593 100.334315) (end 156.680593 102.6023) (width 0.2) (layer "F.Cu") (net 5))
 (segment (start 158.078293 104) (end 165.0025 104) (width 0.2) (layer "F.Cu") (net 5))
 (segment (start 154.95 99.1) (end 155.446279 99.1) (width 0.2) (layer "F.Cu") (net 5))
 (segment (start 154.475 98.975) (end 154.825 98.975) (width 0.2) (layer "F.Cu") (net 5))
 (segment (start 165.0025 104) (end 168.5 100.5025) (width 0.2) (layer "F.Cu") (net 5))
 (segment (start 153.96 98.85) (end 154.35 98.85) (width 0.2) (layer "F.Cu") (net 5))
 (segment (start 154.35 98.85) (end 154.475 98.975) (width 0.2) (layer "F.Cu") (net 5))
 (segment (start 165.168186 104.4) (end 157.912608 104.4) (width 0.2) (layer "F.Cu") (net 6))
 (segment (start 166.534858 103.458359) (end 166.702979 103.62648) (width 0.2) (layer "F.Cu") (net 6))
 (segment (start 157.912608 104.4) (end 156.280593 102.767985) (width 0.2) (layer "F.Cu") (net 6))
 (segment (start 166.534093 103.458359) (end 166.534858 103.458359) (width 0.2) (layer "F.Cu") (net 6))
 (segment (start 156.280593 102.767985) (end 156.280593 100.5) (width 0.2) (layer "F.Cu") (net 6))
 (segment (start 165.685565 103.882624) (end 165.685564 103.882623) (width 0.2) (layer "F.Cu") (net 6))
 (segment (start 166.278715 104.050744) (end 166.276206 104.050744) (width 0.2) (layer "F.Cu") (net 6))
 (segment (start 167.023186 102.545) (end 166.534093 103.034093) (width 0.2) (layer "F.Cu") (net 6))
 (segment (start 155.280593 99.5) (end 153.96 99.5) (width 0.2) (layer "F.Cu") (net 6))
 (segment (start 168.5 102.545) (end 167.023186 102.545) (width 0.2) (layer "F.Cu") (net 6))
 (segment (start 165.685564 103.882623) (end 165.168186 104.4) (width 0.2) (layer "F.Cu") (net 6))
 (segment (start 156.280593 100.5) (end 155.280593 99.5) (width 0.2) (layer "F.Cu") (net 6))
 (segment (start 166.276206 104.050744) (end 166.075497 103.850035) (width 0.2) (layer "F.Cu") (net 6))
 (arc (start 166.075497 103.850035) (mid 165.874159 103.795681) (end 165.685565 103.882624) (width 0.2) (layer "F.Cu") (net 6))
 (arc (start 166.702979 103.62648) (mid 166.790847 103.838612) (end 166.702979 104.050744) (width 0.2) (layer "F.Cu") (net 6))
 (arc (start 166.534093 103.034093) (mid 166.446224 103.246227) (end 166.534093 103.458359) (width 0.2) (layer "F.Cu") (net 6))
 (arc (start 166.702979 104.050744) (mid 166.490847 104.138612) (end 166.278715 104.050744) (width 0.2) (layer "F.Cu") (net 6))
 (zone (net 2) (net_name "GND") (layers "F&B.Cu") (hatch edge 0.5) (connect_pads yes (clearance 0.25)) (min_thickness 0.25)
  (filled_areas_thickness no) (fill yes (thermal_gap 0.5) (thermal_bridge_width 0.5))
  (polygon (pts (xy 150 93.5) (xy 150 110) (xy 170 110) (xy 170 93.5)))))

